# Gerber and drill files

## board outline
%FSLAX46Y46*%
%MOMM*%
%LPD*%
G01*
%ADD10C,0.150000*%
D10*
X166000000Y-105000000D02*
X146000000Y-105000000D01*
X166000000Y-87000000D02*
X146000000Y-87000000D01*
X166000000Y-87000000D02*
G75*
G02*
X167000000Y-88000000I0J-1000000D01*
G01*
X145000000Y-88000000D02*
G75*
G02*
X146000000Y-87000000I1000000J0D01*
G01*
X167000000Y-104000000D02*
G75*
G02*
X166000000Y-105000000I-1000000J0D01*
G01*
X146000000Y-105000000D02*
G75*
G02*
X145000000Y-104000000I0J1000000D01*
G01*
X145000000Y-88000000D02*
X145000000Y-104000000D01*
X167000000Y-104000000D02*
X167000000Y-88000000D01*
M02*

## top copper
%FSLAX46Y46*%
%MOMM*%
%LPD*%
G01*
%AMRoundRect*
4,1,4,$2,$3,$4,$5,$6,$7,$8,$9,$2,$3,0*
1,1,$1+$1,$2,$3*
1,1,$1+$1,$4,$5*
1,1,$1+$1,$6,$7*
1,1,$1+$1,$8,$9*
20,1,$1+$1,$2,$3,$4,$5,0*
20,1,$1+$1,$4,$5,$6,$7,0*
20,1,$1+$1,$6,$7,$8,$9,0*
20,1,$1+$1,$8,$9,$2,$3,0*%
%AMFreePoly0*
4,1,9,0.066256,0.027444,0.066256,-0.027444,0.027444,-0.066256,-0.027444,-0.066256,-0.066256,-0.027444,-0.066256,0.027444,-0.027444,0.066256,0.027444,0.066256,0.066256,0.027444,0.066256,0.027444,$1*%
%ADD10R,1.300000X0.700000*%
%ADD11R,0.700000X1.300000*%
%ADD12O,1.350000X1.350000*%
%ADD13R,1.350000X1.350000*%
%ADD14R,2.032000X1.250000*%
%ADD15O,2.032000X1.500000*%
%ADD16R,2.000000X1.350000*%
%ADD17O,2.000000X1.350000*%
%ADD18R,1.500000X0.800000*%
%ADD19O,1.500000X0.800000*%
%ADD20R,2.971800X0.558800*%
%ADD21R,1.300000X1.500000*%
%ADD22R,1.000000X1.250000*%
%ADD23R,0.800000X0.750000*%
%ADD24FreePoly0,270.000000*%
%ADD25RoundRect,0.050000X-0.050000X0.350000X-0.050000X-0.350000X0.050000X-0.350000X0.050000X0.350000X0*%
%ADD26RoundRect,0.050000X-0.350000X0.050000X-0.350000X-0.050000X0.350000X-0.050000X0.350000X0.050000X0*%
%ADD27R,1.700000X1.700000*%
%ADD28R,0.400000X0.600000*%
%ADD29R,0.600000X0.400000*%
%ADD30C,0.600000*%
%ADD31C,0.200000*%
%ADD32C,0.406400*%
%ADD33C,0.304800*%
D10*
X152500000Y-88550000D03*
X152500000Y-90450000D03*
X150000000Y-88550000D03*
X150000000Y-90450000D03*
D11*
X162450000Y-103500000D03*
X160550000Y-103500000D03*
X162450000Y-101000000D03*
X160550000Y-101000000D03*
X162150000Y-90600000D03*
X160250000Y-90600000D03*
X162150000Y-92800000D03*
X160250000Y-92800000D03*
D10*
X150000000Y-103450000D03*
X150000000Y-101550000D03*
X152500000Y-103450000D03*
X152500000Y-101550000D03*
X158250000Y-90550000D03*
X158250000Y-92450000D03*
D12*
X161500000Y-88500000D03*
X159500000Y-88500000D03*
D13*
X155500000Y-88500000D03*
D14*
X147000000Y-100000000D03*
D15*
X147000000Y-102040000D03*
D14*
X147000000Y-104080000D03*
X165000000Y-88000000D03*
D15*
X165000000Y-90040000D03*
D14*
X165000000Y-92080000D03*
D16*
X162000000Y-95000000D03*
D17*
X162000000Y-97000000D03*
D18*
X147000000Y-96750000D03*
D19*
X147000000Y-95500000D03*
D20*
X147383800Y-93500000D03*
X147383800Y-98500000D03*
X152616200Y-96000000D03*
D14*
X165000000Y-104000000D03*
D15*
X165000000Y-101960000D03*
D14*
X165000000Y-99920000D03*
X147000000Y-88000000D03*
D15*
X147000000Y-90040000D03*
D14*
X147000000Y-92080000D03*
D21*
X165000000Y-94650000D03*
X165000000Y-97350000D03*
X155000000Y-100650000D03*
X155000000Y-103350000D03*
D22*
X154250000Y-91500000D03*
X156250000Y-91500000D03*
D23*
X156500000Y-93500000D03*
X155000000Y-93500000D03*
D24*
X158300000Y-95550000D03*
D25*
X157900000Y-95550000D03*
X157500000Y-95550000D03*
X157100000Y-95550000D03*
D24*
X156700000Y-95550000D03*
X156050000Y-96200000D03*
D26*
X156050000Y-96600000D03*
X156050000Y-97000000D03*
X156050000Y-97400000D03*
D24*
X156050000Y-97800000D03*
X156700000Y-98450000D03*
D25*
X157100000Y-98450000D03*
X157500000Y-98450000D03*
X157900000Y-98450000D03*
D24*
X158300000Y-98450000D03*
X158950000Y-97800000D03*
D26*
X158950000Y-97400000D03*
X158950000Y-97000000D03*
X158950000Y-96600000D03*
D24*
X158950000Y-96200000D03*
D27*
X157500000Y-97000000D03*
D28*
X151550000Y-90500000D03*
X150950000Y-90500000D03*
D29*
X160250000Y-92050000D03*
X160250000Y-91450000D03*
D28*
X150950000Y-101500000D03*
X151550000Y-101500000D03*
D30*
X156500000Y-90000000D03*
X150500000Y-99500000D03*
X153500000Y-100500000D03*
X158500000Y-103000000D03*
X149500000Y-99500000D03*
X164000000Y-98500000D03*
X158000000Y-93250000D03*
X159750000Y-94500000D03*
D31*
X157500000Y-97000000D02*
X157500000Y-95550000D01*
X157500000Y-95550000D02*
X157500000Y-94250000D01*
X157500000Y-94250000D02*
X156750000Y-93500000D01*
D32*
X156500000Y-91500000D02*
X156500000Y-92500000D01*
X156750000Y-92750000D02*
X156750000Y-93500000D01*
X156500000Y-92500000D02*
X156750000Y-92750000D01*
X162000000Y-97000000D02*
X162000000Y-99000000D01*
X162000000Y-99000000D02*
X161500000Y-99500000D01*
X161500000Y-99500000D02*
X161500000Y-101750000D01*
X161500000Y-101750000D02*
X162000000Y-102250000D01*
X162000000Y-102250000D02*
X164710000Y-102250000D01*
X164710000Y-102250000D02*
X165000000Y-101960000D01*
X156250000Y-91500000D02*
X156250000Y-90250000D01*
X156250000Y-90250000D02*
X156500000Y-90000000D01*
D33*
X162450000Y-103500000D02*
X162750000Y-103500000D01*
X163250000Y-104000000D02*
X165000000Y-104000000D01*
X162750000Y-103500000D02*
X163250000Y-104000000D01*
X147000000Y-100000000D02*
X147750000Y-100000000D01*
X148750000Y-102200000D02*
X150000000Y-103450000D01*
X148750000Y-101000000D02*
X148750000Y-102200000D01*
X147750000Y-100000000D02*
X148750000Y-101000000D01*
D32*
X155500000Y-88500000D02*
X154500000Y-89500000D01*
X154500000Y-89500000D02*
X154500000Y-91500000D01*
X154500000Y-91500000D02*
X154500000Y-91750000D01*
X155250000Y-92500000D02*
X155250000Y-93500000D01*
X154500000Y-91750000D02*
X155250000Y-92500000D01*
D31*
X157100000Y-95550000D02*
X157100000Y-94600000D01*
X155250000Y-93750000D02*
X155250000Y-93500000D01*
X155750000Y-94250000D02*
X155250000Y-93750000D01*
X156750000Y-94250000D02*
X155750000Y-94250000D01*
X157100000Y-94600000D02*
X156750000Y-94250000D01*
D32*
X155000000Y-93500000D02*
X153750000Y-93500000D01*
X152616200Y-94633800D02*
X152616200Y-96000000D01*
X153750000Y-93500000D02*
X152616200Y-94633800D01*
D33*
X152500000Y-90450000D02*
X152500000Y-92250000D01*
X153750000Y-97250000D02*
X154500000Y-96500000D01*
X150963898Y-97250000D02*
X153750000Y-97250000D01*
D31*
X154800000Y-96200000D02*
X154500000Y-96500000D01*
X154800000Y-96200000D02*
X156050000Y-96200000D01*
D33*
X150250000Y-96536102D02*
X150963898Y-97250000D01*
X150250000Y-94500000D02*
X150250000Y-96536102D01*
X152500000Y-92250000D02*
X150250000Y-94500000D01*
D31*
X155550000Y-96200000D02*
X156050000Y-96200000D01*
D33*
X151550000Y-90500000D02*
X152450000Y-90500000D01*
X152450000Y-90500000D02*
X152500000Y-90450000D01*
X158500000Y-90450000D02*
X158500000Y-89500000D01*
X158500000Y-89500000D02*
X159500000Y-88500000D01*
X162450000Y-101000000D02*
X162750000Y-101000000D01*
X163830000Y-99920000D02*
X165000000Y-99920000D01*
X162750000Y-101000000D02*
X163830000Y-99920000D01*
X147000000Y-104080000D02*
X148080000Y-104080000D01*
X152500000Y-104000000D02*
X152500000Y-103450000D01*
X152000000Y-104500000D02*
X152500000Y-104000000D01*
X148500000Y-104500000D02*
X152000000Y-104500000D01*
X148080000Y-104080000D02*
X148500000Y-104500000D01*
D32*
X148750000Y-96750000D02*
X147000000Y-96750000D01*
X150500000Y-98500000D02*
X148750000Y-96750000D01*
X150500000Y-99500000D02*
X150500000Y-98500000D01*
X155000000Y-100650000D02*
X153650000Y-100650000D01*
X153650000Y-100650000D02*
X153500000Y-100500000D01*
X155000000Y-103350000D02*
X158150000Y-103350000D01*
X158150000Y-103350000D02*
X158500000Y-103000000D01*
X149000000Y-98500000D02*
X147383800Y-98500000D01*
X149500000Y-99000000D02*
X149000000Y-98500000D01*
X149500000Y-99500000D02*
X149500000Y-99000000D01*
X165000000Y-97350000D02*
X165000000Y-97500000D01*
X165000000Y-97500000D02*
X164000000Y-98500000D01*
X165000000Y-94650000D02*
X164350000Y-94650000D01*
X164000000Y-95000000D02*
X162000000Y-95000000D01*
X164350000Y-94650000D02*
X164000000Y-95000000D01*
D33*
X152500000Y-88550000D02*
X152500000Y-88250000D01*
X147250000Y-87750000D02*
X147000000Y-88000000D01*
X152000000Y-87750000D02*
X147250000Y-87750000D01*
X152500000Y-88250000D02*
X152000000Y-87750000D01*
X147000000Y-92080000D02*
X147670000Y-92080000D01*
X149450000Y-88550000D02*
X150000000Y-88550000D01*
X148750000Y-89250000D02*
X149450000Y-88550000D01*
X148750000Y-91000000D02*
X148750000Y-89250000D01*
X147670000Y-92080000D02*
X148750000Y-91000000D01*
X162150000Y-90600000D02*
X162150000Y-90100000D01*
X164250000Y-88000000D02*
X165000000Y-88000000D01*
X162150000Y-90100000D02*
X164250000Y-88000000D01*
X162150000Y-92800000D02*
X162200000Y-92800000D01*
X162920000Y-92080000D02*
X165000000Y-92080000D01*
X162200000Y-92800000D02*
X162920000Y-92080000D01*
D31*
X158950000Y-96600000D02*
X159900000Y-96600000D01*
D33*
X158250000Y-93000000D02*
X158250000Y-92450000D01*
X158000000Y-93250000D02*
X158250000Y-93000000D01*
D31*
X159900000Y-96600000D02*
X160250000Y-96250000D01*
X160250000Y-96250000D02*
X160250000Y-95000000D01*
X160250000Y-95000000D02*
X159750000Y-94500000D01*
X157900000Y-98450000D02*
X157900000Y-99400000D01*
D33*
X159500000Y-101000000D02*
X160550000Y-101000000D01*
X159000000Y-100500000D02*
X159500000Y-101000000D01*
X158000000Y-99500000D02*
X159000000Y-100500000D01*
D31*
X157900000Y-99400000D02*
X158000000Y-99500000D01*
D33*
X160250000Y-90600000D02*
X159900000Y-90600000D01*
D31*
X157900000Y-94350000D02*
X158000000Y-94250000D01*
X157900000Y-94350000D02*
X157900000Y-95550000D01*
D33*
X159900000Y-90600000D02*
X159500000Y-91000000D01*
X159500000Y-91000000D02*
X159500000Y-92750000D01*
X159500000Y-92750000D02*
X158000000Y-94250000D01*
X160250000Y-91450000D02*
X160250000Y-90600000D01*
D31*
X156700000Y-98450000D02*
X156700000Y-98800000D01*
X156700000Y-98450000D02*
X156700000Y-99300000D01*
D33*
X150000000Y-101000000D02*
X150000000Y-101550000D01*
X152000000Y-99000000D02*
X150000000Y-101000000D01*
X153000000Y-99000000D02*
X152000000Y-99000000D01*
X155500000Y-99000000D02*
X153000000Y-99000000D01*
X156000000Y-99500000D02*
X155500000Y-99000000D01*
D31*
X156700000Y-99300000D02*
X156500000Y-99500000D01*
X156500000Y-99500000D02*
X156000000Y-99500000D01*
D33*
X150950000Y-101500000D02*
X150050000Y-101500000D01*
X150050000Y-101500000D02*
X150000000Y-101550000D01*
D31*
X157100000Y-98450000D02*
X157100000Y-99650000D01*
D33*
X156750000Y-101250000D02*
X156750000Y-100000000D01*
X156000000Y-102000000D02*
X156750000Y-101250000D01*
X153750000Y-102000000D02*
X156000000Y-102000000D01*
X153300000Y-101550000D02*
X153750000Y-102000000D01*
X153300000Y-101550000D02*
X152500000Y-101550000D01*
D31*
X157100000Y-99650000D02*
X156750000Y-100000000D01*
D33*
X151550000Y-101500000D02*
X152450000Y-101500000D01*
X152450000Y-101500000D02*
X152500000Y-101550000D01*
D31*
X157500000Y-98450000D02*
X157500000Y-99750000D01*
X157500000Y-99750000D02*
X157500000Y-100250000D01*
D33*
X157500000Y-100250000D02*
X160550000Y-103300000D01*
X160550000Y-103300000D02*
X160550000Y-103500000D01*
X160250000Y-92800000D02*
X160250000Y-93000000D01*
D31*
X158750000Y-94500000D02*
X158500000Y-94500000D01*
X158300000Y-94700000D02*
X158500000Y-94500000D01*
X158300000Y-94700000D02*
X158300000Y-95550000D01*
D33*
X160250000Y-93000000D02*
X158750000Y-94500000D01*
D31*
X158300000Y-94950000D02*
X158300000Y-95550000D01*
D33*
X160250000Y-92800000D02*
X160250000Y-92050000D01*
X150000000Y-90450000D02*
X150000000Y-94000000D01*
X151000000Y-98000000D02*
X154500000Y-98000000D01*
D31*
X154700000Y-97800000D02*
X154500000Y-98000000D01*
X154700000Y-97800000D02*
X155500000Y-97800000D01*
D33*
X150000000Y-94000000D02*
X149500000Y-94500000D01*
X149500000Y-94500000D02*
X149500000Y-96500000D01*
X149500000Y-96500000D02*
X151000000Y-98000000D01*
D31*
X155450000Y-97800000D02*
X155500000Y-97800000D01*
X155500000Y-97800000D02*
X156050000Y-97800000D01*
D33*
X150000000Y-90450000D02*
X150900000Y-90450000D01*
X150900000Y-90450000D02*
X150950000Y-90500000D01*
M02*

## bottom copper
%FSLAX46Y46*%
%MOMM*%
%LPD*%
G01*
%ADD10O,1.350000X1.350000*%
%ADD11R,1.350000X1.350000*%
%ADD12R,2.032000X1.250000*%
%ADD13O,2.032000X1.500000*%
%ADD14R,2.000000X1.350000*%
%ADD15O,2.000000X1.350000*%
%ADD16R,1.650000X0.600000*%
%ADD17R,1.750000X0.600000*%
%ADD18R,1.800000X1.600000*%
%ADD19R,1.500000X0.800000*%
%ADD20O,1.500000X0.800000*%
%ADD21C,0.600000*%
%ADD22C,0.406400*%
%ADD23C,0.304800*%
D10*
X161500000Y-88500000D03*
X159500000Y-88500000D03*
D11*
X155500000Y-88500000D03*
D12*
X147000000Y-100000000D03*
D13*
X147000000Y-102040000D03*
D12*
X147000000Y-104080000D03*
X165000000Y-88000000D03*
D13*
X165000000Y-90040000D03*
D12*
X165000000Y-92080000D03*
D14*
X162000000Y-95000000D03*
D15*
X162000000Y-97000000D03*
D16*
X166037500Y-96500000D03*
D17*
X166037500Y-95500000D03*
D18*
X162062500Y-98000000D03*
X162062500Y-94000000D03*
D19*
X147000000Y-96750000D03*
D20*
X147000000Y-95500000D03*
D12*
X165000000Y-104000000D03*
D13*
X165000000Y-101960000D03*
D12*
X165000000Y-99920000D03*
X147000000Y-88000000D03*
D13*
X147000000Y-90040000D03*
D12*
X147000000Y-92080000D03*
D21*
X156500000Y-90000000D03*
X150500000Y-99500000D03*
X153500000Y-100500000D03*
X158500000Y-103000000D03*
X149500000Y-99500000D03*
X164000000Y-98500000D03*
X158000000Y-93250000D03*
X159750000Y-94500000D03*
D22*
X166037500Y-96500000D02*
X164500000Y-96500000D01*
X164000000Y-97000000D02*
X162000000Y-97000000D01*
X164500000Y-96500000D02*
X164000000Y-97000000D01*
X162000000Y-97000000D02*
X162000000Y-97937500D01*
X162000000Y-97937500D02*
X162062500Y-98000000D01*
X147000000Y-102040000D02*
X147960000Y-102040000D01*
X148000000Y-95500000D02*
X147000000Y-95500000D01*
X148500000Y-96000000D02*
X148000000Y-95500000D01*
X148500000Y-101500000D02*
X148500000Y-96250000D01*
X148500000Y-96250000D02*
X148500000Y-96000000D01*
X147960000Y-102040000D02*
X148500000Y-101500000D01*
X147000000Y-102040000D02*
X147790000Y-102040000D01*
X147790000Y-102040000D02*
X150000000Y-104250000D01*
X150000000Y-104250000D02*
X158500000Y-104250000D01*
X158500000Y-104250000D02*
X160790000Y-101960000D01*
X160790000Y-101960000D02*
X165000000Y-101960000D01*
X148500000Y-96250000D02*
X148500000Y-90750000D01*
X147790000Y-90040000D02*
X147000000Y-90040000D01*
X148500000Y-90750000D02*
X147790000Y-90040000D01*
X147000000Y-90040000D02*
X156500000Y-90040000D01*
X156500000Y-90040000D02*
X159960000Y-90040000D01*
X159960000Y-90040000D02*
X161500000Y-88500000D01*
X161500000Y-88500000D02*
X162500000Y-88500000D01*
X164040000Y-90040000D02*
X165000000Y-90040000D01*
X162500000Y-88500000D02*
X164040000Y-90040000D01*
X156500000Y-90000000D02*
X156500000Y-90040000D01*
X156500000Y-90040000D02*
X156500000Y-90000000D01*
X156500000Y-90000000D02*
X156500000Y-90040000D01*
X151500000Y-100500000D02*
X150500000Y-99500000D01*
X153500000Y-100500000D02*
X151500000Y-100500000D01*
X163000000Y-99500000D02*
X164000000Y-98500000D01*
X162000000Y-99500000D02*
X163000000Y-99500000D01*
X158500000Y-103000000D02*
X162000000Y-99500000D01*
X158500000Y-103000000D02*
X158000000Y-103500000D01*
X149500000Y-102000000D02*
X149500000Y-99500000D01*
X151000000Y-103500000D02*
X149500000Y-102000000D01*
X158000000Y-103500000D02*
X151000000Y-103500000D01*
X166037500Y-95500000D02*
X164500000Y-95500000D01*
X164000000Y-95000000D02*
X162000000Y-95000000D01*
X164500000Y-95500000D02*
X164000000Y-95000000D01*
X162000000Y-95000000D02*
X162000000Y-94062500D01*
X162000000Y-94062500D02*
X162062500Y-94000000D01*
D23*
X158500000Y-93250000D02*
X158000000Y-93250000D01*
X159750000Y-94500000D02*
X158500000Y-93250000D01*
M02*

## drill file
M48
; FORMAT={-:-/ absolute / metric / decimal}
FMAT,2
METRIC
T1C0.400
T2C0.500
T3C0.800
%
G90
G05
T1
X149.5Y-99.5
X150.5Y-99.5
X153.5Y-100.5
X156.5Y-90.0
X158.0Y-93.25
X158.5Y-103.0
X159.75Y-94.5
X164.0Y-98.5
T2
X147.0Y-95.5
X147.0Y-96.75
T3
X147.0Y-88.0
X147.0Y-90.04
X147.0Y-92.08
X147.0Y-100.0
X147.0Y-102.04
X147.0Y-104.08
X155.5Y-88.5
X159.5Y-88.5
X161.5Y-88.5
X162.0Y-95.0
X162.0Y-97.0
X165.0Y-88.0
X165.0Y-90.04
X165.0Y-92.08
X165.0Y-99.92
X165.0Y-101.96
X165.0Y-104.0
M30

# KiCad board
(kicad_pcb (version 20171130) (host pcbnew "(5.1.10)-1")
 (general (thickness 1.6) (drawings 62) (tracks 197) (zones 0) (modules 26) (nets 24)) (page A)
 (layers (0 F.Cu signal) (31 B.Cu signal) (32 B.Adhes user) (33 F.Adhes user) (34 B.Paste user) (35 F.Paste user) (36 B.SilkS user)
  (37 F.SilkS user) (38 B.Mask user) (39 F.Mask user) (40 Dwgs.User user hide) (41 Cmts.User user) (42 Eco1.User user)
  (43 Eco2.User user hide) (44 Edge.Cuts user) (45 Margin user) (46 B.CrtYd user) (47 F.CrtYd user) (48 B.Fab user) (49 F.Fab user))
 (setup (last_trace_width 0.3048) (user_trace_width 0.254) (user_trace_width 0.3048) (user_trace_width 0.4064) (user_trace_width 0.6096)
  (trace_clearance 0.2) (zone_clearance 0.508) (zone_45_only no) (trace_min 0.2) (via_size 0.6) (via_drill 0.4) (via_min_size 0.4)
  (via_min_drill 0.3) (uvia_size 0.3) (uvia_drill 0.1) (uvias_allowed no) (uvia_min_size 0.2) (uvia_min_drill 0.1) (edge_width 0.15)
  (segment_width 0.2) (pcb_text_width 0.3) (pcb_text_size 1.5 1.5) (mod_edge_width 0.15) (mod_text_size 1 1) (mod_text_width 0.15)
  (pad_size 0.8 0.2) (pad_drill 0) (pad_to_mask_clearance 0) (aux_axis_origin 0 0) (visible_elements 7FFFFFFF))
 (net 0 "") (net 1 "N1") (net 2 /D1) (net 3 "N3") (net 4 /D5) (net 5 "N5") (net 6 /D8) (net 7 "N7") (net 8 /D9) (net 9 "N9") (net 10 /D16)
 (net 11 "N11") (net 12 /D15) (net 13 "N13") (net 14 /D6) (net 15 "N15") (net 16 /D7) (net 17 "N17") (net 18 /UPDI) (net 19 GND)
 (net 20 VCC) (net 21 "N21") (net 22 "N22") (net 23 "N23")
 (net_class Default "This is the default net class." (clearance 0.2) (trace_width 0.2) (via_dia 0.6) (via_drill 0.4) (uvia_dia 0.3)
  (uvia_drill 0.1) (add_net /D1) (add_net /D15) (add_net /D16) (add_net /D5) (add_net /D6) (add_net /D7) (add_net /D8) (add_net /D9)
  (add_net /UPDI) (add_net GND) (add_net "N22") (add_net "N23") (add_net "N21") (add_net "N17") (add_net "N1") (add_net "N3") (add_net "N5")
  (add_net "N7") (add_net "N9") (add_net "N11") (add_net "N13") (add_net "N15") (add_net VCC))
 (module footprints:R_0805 (layer F.Cu) (at 152.5 89.5 90)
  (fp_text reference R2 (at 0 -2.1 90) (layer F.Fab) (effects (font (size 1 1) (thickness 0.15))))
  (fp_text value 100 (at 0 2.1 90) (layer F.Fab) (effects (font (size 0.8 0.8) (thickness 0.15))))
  (pad 2 smd rect (at 0.95 0 90) (size 0.7 1.3) (layers F.Cu F.Paste F.Mask) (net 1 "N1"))
  (pad 1 smd rect (at -0.95 0 90) (size 0.7 1.3) (layers F.Cu F.Paste F.Mask) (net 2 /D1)))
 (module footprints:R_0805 (layer F.Cu) (at 150 89.5 90)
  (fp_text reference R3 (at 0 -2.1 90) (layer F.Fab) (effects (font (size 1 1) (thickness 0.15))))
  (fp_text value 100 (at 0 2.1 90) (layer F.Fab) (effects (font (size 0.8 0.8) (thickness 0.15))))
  (pad 2 smd rect (at 0.95 0 90) (size 0.7 1.3) (layers F.Cu F.Paste F.Mask) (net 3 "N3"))
  (pad 1 smd rect (at -0.95 0 90) (size 0.7 1.3) (layers F.Cu F.Paste F.Mask) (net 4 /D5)))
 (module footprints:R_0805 (layer F.Cu) (at 161.5 103.5)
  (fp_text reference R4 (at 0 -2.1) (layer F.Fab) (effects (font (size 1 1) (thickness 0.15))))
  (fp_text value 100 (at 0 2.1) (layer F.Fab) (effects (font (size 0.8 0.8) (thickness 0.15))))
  (pad 2 smd rect (at 0.95 0) (size 0.7 1.3) (layers F.Cu F.Paste F.Mask) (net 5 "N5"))
  (pad 1 smd rect (at -0.95 0) (size 0.7 1.3) (layers F.Cu F.Paste F.Mask) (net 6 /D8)))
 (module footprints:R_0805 (layer F.Cu) (at 161.5 101)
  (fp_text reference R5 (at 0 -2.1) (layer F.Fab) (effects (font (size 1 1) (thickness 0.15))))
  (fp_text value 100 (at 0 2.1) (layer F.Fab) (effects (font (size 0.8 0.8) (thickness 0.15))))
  (pad 2 smd rect (at 0.95 0) (size 0.7 1.3) (layers F.Cu F.Paste F.Mask) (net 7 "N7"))
  (pad 1 smd rect (at -0.95 0) (size 0.7 1.3) (layers F.Cu F.Paste F.Mask) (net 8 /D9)))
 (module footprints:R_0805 (layer F.Cu) (at 161.2 90.6)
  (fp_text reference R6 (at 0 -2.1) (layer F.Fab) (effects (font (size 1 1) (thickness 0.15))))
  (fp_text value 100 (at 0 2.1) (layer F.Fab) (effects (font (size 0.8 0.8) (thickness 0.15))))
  (pad 2 smd rect (at 0.95 0) (size 0.7 1.3) (layers F.Cu F.Paste F.Mask) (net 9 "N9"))
  (pad 1 smd rect (at -0.95 0) (size 0.7 1.3) (layers F.Cu F.Paste F.Mask) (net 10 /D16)))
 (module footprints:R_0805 (layer F.Cu) (at 161.2 92.8)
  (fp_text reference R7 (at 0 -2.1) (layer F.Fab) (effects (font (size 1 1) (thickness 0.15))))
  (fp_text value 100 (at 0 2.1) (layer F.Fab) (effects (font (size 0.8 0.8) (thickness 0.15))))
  (pad 2 smd rect (at 0.95 0) (size 0.7 1.3) (layers F.Cu F.Paste F.Mask) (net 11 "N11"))
  (pad 1 smd rect (at -0.95 0) (size 0.7 1.3) (layers F.Cu F.Paste F.Mask) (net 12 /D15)))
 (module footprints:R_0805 (layer F.Cu) (at 150 102.5 270)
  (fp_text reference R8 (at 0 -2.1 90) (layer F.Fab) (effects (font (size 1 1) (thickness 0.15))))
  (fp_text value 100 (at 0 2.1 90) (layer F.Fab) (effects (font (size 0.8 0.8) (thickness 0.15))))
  (pad 2 smd rect (at 0.95 0 270) (size 0.7 1.3) (layers F.Cu F.Paste F.Mask) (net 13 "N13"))
  (pad 1 smd rect (at -0.95 0 270) (size 0.7 1.3) (layers F.Cu F.Paste F.Mask) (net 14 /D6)))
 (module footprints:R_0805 (layer F.Cu) (at 152.5 102.5 270)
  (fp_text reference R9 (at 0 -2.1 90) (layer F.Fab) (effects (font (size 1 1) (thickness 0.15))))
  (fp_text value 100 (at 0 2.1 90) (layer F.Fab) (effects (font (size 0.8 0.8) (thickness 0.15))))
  (pad 2 smd rect (at 0.95 0 270) (size 0.7 1.3) (layers F.Cu F.Paste F.Mask) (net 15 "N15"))
  (pad 1 smd rect (at -0.95 0 270) (size 0.7 1.3) (layers F.Cu F.Paste F.Mask) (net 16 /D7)))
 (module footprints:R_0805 (layer F.Cu) (at 158.25 91.5 90)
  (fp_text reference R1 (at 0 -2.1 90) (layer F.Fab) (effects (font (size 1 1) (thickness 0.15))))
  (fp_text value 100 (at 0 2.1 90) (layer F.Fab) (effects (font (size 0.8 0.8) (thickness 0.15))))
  (pad 2 smd rect (at 0.95 0 90) (size 0.7 1.3) (layers F.Cu F.Paste F.Mask) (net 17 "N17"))
  (pad 1 smd rect (at -0.95 0 90) (size 0.7 1.3) (layers F.Cu F.Paste F.Mask) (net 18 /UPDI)))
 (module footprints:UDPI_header (layer B.Cu) (at 155.5 88.5 270)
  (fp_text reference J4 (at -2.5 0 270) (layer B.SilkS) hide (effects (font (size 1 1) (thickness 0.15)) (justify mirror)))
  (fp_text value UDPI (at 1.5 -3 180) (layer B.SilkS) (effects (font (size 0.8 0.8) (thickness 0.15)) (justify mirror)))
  (pad 4 thru_hole oval (at 0 -6 270) (size 1.35 1.35) (drill 0.8) (layers *.Cu *.Mask) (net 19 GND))
  (pad 3 thru_hole oval (at 0 -4 270) (size 1.35 1.35) (drill 0.8) (layers *.Cu *.Mask) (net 17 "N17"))
  (pad 1 thru_hole rect (at 0 0 270) (size 1.35 1.35) (drill 0.8) (layers *.Cu *.Mask) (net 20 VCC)))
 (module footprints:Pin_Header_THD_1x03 (layer F.Cu) (at 147 100)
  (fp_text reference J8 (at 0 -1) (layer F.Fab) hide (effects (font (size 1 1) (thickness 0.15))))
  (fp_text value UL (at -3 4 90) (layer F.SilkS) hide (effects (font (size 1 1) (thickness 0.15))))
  (pad 1 thru_hole rect (at 0 0) (size 2.032 1.25) (drill 0.8) (layers *.Cu *.Mask F.SilkS) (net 13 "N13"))
  (pad 2 thru_hole oval (at 0 2.04) (size 2.032 1.5) (drill 0.8) (layers *.Cu *.Mask F.SilkS) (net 19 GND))
  (pad 3 thru_hole rect (at 0 4.08) (size 2.032 1.25) (drill 0.8) (layers *.Cu *.Mask F.SilkS) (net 15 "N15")))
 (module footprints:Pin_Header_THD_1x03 (layer F.Cu) (at 165 88)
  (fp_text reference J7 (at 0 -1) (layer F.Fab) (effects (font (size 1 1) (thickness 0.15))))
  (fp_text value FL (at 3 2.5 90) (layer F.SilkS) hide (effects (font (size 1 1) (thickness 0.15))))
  (pad 1 thru_hole rect (at 0 0) (size 2.032 1.25) (drill 0.8) (layers *.Cu *.Mask F.SilkS) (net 9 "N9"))
  (pad 2 thru_hole oval (at 0 2.04) (size 2.032 1.5) (drill 0.8) (layers *.Cu *.Mask F.SilkS) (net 19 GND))
  (pad 3 thru_hole rect (at 0 4.08) (size 2.032 1.25) (drill 0.8) (layers *.Cu *.Mask F.SilkS) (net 11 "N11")))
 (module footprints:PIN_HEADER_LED (layer B.Cu) (at 162 95 180)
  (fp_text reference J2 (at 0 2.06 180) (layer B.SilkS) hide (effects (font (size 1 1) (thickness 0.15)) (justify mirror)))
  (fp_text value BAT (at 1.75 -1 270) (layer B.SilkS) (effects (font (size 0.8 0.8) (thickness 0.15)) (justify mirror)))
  (pad 1 thru_hole rect (at 0 0 180) (size 2 1.35) (drill 0.8) (layers *.Cu *.Mask) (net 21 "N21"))
  (pad 2 thru_hole oval (at 0 -2 180) (size 2 1.35) (drill 0.8) (layers *.Cu *.Mask) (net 19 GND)))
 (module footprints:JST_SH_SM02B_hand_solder (layer B.Cu) (at 164 96 90)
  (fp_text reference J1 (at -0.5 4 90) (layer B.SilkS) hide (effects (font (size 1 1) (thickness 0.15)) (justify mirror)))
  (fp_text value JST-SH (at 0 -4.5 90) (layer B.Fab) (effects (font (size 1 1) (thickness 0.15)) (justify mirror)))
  (pad 1 smd rect (at -0.5 2.0375 90) (size 0.6 1.65) (layers B.Cu B.Paste B.Mask) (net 19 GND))
  (pad 2 smd rect (at 0.5 2.0375 90) (size 0.6 1.75) (layers B.Cu B.Paste B.Mask) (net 21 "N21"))
  (pad 1 smd rect (at -2 -1.9375 90) (size 1.6 1.8) (layers B.Cu B.Paste B.Mask) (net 19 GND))
  (pad 2 smd rect (at 2 -1.9375 90) (size 1.6 1.8) (layers B.Cu B.Paste B.Mask) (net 21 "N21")))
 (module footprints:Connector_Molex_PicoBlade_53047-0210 (layer F.Cu) (at 147 96.75 90)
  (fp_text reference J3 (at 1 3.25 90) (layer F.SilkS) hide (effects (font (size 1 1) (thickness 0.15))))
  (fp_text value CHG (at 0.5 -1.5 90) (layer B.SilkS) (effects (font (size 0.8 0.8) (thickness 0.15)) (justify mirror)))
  (pad 1 thru_hole rect (at 0 0 90) (size 0.8 1.5) (drill 0.5) (layers *.Cu *.Mask F.SilkS) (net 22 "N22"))
  (pad 2 thru_hole oval (at 1.25 0 90) (size 0.8 1.5) (drill 0.5) (layers *.Cu *.Mask F.SilkS) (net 19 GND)))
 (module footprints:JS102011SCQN (layer F.Cu) (at 150 96)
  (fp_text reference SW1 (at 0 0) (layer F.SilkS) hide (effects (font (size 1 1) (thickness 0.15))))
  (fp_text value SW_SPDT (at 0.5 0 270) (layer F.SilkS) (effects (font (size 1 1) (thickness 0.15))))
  (pad 1 smd rect (at -2.6162 -2.5) (size 2.9718 0.5588) (layers F.Cu F.Paste F.Mask))
  (pad 3 smd rect (at -2.6162 2.5) (size 2.9718 0.5588) (layers F.Cu F.Paste F.Mask) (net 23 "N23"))
  (pad 2 smd rect (at 2.6162 0) (size 2.9718 0.5588) (layers F.Cu F.Paste F.Mask) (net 20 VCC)))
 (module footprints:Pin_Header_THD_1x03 (layer F.Cu) (at 165 104 180)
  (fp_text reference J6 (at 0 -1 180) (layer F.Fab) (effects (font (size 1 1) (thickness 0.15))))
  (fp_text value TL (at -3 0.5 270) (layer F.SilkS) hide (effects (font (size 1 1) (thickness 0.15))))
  (pad 1 thru_hole rect (at 0 0 180) (size 2.032 1.25) (drill 0.8) (layers *.Cu *.Mask F.SilkS) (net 5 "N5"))
  (pad 2 thru_hole oval (at 0 2.04 180) (size 2.032 1.5) (drill 0.8) (layers *.Cu *.Mask F.SilkS) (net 19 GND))
  (pad 3 thru_hole rect (at 0 4.08 180) (size 2.032 1.25) (drill 0.8) (layers *.Cu *.Mask F.SilkS) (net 7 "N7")))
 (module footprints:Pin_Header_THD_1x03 (layer F.Cu) (at 147 88)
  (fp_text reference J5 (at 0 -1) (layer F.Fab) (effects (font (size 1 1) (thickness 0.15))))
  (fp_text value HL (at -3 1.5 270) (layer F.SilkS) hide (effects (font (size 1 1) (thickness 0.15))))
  (pad 1 thru_hole rect (at 0 0) (size 2.032 1.25) (drill 0.8) (layers *.Cu *.Mask F.SilkS) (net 1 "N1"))
  (pad 2 thru_hole oval (at 0 2.04) (size 2.032 1.5) (drill 0.8) (layers *.Cu *.Mask F.SilkS) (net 19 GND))
  (pad 3 thru_hole rect (at 0 4.08) (size 2.032 1.25) (drill 0.8) (layers *.Cu *.Mask F.SilkS) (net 3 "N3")))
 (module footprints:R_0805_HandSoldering (layer F.Cu) (at 165 96 270)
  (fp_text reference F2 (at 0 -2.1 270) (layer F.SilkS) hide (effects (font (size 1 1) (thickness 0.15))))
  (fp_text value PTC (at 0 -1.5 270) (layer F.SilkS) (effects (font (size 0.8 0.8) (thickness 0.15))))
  (pad 1 smd rect (at -1.35 0 270) (size 1.5 1.3) (layers F.Cu F.Paste F.Mask) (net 21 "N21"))
  (pad 2 smd rect (at 1.35 0 270) (size 1.5 1.3) (layers F.Cu F.Paste F.Mask) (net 23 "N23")))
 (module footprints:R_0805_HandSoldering (layer F.Cu) (at 155 102 270)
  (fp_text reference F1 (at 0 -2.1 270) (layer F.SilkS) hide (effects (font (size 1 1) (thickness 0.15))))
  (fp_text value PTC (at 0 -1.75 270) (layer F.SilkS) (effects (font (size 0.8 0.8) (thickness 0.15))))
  (pad 1 smd rect (at -1.35 0 270) (size 1.5 1.3) (layers F.Cu F.Paste F.Mask) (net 22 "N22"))
  (pad 2 smd rect (at 1.35 0 270) (size 1.5 1.3) (layers F.Cu F.Paste F.Mask) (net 23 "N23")))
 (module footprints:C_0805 (layer F.Cu) (at 155.25 91.5)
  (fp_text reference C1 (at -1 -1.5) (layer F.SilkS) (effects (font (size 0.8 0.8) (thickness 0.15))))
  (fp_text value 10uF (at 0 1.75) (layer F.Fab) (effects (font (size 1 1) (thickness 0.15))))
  (pad 1 smd rect (at -1 0) (size 1 1.25) (layers F.Cu F.Paste F.Mask) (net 20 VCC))
  (pad 2 smd rect (at 1 0) (size 1 1.25) (layers F.Cu F.Paste F.Mask) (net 19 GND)))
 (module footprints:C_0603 (layer F.Cu) (at 155.75 93.5)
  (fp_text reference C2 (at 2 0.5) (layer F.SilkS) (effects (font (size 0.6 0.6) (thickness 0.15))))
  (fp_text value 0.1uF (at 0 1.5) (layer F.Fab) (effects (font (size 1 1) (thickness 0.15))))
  (pad 2 smd rect (at 0.75 0) (size 0.8 0.75) (layers F.Cu F.Paste F.Mask) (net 19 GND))
  (pad 1 smd rect (at -0.75 0) (size 0.8 0.75) (layers F.Cu F.Paste F.Mask) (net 20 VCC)))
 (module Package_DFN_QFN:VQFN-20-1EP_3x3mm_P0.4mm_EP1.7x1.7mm (layer F.Cu) (at 157.5 97 270)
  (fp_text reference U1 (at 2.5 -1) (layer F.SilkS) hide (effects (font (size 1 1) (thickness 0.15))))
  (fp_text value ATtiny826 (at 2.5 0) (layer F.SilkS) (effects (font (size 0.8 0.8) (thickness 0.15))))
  (pad 1 smd custom (at -1.45 -0.8 270) (size 0.143431 0.143431) (layers F.Cu F.Paste F.Mask) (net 12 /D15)
   (options (clearance outline) (anchor circle)) (primitives))
  (pad 2 smd roundrect (at -1.45 -0.4 270) (size 0.8 0.2) (layers F.Cu F.Paste F.Mask) (roundrect_rratio 0.25) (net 10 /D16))
  (pad 3 smd roundrect (at -1.45 0 270) (size 0.8 0.2) (layers F.Cu F.Paste F.Mask) (roundrect_rratio 0.25) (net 19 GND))
  (pad 4 smd roundrect (at -1.45 0.4 270) (size 0.8 0.2) (layers F.Cu F.Paste F.Mask) (roundrect_rratio 0.25) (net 20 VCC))
  (pad 5 smd custom (at -1.45 0.8 270) (size 0.143431 0.143431) (layers F.Cu F.Paste F.Mask) (options (clearance outline) (anchor circle))
   (primitives))
  (pad 6 smd custom (at -0.8 1.45 270) (size 0.143431 0.143431) (layers F.Cu F.Paste F.Mask) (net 2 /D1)
   (options (clearance outline) (anchor circle)) (primitives))
  (pad 7 smd roundrect (at -0.4 1.45 270) (size 0.2 0.8) (layers F.Cu F.Paste F.Mask) (roundrect_rratio 0.25))
  (pad 8 smd roundrect (at 0 1.45 270) (size 0.2 0.8) (layers F.Cu F.Paste F.Mask) (roundrect_rratio 0.25))
  (pad 9 smd roundrect (at 0.4 1.45 270) (size 0.2 0.8) (layers F.Cu F.Paste F.Mask) (roundrect_rratio 0.25))
  (pad 10 smd custom (at 0.8 1.45 270) (size 0.143431 0.143431) (layers F.Cu F.Paste F.Mask) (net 4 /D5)
   (options (clearance outline) (anchor circle)) (primitives))
  (pad 11 smd custom (at 1.45 0.8 270) (size 0.143431 0.143431) (layers F.Cu F.Paste F.Mask) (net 14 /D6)
   (options (clearance outline) (anchor circle)) (primitives))
  (pad 12 smd roundrect (at 1.45 0.4 270) (size 0.8 0.2) (layers F.Cu F.Paste F.Mask) (roundrect_rratio 0.25) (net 16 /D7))
  (pad 13 smd roundrect (at 1.45 0 270) (size 0.8 0.2) (layers F.Cu F.Paste F.Mask) (roundrect_rratio 0.25) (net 6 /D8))
  (pad 14 smd roundrect (at 1.45 -0.4 270) (size 0.8 0.2) (layers F.Cu F.Paste F.Mask) (roundrect_rratio 0.25) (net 8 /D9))
  (pad 15 smd custom (at 1.45 -0.8 270) (size 0.143431 0.143431) (layers F.Cu F.Paste F.Mask) (options (clearance outline) (anchor circle))
   (primitives))
  (pad 16 smd custom (at 0.8 -1.45 270) (size 0.143431 0.143431) (layers F.Cu F.Paste F.Mask) (options (clearance outline) (anchor circle))
   (primitives))
  (pad 17 smd roundrect (at 0.4 -1.45 270) (size 0.2 0.8) (layers F.Cu F.Paste F.Mask) (roundrect_rratio 0.25))
  (pad 18 smd roundrect (at 0 -1.45 270) (size 0.2 0.8) (layers F.Cu F.Paste F.Mask) (roundrect_rratio 0.25))
  (pad 19 smd roundrect (at -0.4 -1.45 270) (size 0.2 0.8) (layers F.Cu F.Paste F.Mask) (roundrect_rratio 0.25) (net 18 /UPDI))
  (pad 20 smd custom (at -0.8 -1.45 270) (size 0.143431 0.143431) (layers F.Cu F.Paste F.Mask) (options (clearance outline) (anchor circle))
   (primitives))
  (pad 21 smd rect (at 0 0 270) (size 1.7 1.7) (layers F.Cu F.Mask) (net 19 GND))
  (pad "" smd roundrect (at -0.425 -0.425 270) (size 0.69 0.69) (layers F.Paste) (roundrect_rratio 0.25))
  (pad "" smd roundrect (at -0.425 0.425 270) (size 0.69 0.69) (layers F.Paste) (roundrect_rratio 0.25))
  (pad "" smd roundrect (at 0.425 -0.425 270) (size 0.69 0.69) (layers F.Paste) (roundrect_rratio 0.25))
  (pad "" smd roundrect (at 0.425 0.425 270) (size 0.69 0.69) (layers F.Paste) (roundrect_rratio 0.25)))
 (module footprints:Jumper (layer F.Cu) (at 151.25 90.5 180)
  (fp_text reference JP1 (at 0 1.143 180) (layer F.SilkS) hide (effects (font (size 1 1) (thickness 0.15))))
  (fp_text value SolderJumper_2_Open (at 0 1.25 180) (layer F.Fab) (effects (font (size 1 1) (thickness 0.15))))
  (pad 1 smd rect (at -0.3 0 180) (size 0.4 0.6) (layers F.Cu F.Paste F.Mask) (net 2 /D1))
  (pad 2 smd rect (at 0.3 0 180) (size 0.4 0.6) (layers F.Cu F.Paste F.Mask) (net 4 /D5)))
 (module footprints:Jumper (layer F.Cu) (at 160.25 91.75 270)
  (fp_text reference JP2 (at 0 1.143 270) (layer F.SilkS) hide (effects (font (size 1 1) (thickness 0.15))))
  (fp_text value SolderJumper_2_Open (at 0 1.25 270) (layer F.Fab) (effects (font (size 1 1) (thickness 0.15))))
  (pad 2 smd rect (at 0.3 0 270) (size 0.4 0.6) (layers F.Cu F.Paste F.Mask) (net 12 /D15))
  (pad 1 smd rect (at -0.3 0 270) (size 0.4 0.6) (layers F.Cu F.Paste F.Mask) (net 10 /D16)))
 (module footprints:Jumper (layer F.Cu) (at 151.25 101.5)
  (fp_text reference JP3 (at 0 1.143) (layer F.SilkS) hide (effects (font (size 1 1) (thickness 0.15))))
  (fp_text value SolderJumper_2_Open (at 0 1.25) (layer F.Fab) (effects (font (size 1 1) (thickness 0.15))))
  (pad 1 smd rect (at -0.3 0) (size 0.4 0.6) (layers F.Cu F.Paste F.Mask) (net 14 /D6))
  (pad 2 smd rect (at 0.3 0) (size 0.4 0.6) (layers F.Cu F.Paste F.Mask) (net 16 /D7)))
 (gr_line (start 166 105) (end 146 105) (angle 90) (layer Edge.Cuts) (width 0.15))
 (gr_line (start 166 87) (end 146 87) (angle 90) (layer Edge.Cuts) (width 0.15))
 (gr_arc (start 166 88) (end 166 87) (angle 90) (layer Edge.Cuts) (width 0.15))
 (gr_arc (start 146 88) (end 145 88) (angle 90) (layer Edge.Cuts) (width 0.15))
 (gr_arc (start 166 104) (end 167 104) (angle 90) (layer Edge.Cuts) (width 0.15))
 (gr_arc (start 146 104) (end 146 105) (angle 90) (layer Edge.Cuts) (width 0.15))
 (gr_line (start 145 88) (end 145 104) (angle 90) (layer Edge.Cuts) (width 0.15))
 (gr_line (start 167 104) (end 167 88) (angle 90) (layer Edge.Cuts) (width 0.15))
 (segment (start 166.0375 96.5) (end 164.5 96.5) (width 0.4064) (layer B.Cu) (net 19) (status 400010))
 (segment (start 164 97) (end 162 97) (width 0.4064) (layer B.Cu) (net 19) (status 800020))
 (segment (start 164.5 96.5) (end 164 97) (width 0.4064) (layer B.Cu) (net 19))
 (segment (start 162 97) (end 162 97.9375) (width 0.4064) (layer B.Cu) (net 19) (status C00030))
 (segment (start 162 97.9375) (end 162.0625 98) (width 0.4064) (layer B.Cu) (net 19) (status C00030))
 (segment (start 147 102.04) (end 147.96 102.04) (width 0.4064) (layer B.Cu) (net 19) (status C00030))
 (segment (start 148 95.5) (end 147 95.5) (width 0.4064) (layer B.Cu) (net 19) (status 800020))
 (segment (start 148.5 96) (end 148 95.5) (width 0.4064) (layer B.Cu) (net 19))
 (segment (start 148.5 101.5) (end 148.5 96.25) (width 0.4064) (layer B.Cu) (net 19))
 (segment (start 148.5 96.25) (end 148.5 96) (width 0.4064) (layer B.Cu) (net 19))
 (segment (start 147.96 102.04) (end 148.5 101.5) (width 0.4064) (layer B.Cu) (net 19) (status 400010))
 (segment (start 147 102.04) (end 147.79 102.04) (width 0.4064) (layer B.Cu) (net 19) (status C00030))
 (segment (start 147.79 102.04) (end 150 104.25) (width 0.4064) (layer B.Cu) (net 19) (status 400010))
 (segment (start 150 104.25) (end 158.5 104.25) (width 0.4064) (layer B.Cu) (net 19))
 (segment (start 158.5 104.25) (end 160.79 101.96) (width 0.4064) (layer B.Cu) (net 19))
 (segment (start 160.79 101.96) (end 165 101.96) (width 0.4064) (layer B.Cu) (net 19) (status 800020))
 (segment (start 148.5 96.25) (end 148.5 90.75) (width 0.4064) (layer B.Cu) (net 19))
 (segment (start 147.79 90.04) (end 147 90.04) (width 0.4064) (layer B.Cu) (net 19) (status C00030))
 (segment (start 148.5 90.75) (end 147.79 90.04) (width 0.4064) (layer B.Cu) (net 19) (status 800020))
 (segment (start 147 90.04) (end 156.5 90.04) (width 0.4064) (layer B.Cu) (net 19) (status 400010))
 (segment (start 156.5 90.04) (end 159.96 90.04) (width 0.4064) (layer B.Cu) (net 19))
 (segment (start 159.96 90.04) (end 161.5 88.5) (width 0.4064) (layer B.Cu) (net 19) (status 800020))
 (segment (start 161.5 88.5) (end 162.5 88.5) (width 0.4064) (layer B.Cu) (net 19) (status 400010))
 (segment (start 164.04 90.04) (end 165 90.04) (width 0.4064) (layer B.Cu) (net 19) (status C00030))
 (segment (start 162.5 88.5) (end 164.04 90.04) (width 0.4064) (layer B.Cu) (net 19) (status 800020))
 (segment (start 157.5 97) (end 157.5 95.55) (width 0.2) (layer F.Cu) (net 19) (status C00030))
 (segment (start 157.5 95.55) (end 157.5 94.25) (width 0.2) (layer F.Cu) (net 19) (status 400010))
 (segment (start 157.5 94.25) (end 156.75 93.5) (width 0.2) (layer F.Cu) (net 19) (status 800020))
 (segment (start 156.5 91.5) (end 156.5 92.5) (width 0.4064) (layer F.Cu) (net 19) (status 400010))
 (segment (start 156.75 92.75) (end 156.75 93.5) (width 0.4064) (layer F.Cu) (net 19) (status 800020))
 (segment (start 156.5 92.5) (end 156.75 92.75) (width 0.4064) (layer F.Cu) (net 19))
 (segment (start 162 97) (end 162 99) (width 0.4064) (layer F.Cu) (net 19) (status 400010))
 (segment (start 162 99) (end 161.5 99.5) (width 0.4064) (layer F.Cu) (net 19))
 (segment (start 161.5 99.5) (end 161.5 101.75) (width 0.4064) (layer F.Cu) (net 19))
 (segment (start 161.5 101.75) (end 162 102.25) (width 0.4064) (layer F.Cu) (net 19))
 (segment (start 162 102.25) (end 164.71 102.25) (width 0.4064) (layer F.Cu) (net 19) (status 800020))
 (segment (start 164.71 102.25) (end 165 101.96) (width 0.4064) (layer F.Cu) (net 19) (status C00030))
 (segment (start 156.25 91.5) (end 156.25 90.25) (width 0.4064) (layer F.Cu) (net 19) (status 400010))
 (via (at 156.5 90) (size 0.6) (drill 0.4) (layers F.Cu B.Cu) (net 19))
 (segment (start 156.25 90.25) (end 156.5 90) (width 0.4064) (layer F.Cu) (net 19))
 (segment (start 156.5 90) (end 156.5 90.04) (width 0.4064) (layer B.Cu) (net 19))
 (segment (start 156.5 90.04) (end 156.5 90) (width 0.4064) (layer B.Cu) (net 19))
 (segment (start 156.5 90) (end 156.5 90.04) (width 0.4064) (layer B.Cu) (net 19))
 (segment (start 162.45 103.5) (end 162.75 103.5) (width 0.3048) (layer F.Cu) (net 5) (status C00030))
 (segment (start 163.25 104) (end 165 104) (width 0.3048) (layer F.Cu) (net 5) (status 800020))
 (segment (start 162.75 103.5) (end 163.25 104) (width 0.3048) (layer F.Cu) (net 5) (status 400010))
 (segment (start 147 100) (end 147.75 100) (width 0.3048) (layer F.Cu) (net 13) (status C00030))
 (segment (start 148.75 102.2) (end 150 103.45) (width 0.3048) (layer F.Cu) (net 13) (status 800020))
 (segment (start 148.75 101) (end 148.75 102.2) (width 0.3048) (layer F.Cu) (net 13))
 (segment (start 147.75 100) (end 148.75 101) (width 0.3048) (layer F.Cu) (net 13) (status 400010))
 (segment (start 155.5 88.5) (end 154.5 89.5) (width 0.4064) (layer F.Cu) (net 20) (status 400010))
 (segment (start 154.5 89.5) (end 154.5 91.5) (width 0.4064) (layer F.Cu) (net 20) (status 800020))
 (segment (start 154.5 91.5) (end 154.5 91.75) (width 0.4064) (layer F.Cu) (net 20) (status C00030))
 (segment (start 155.25 92.5) (end 155.25 93.5) (width 0.4064) (layer F.Cu) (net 20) (status 800020))
 (segment (start 154.5 91.75) (end 155.25 92.5) (width 0.4064) (layer F.Cu) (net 20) (status 400010))
 (segment (start 157.1 95.55) (end 157.1 94.6) (width 0.2) (layer F.Cu) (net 20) (status 400010))
 (segment (start 155.25 93.75) (end 155.25 93.5) (width 0.2) (layer F.Cu) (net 20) (status C00030))
 (segment (start 155.75 94.25) (end 155.25 93.75) (width 0.2) (layer F.Cu) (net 20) (status 800020))
 (segment (start 156.75 94.25) (end 155.75 94.25) (width 0.2) (layer F.Cu) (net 20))
 (segment (start 157.1 94.6) (end 156.75 94.25) (width 0.2) (layer F.Cu) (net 20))
 (segment (start 155 93.5) (end 153.75 93.5) (width 0.4064) (layer F.Cu) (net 20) (status 400010))
 (segment (start 152.6162 94.6338) (end 152.6162 96) (width 0.4064) (layer F.Cu) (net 20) (status 800020))
 (segment (start 153.75 93.5) (end 152.6162 94.6338) (width 0.4064) (layer F.Cu) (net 20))
 (segment (start 152.5 90.45) (end 152.5 92.25) (width 0.3048) (layer F.Cu) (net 2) (status 400010))
 (segment (start 153.75 97.25) (end 154.5 96.5) (width 0.3048) (layer F.Cu) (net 2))
 (segment (start 150.963898 97.25) (end 153.75 97.25) (width 0.3048) (layer F.Cu) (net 2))
 (segment (start 154.8 96.2) (end 154.5 96.5) (width 0.2) (layer F.Cu) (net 2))
 (segment (start 154.8 96.2) (end 156.05 96.2) (width 0.2) (layer F.Cu) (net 2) (status 800020))
 (segment (start 150.25 96.536102) (end 150.963898 97.25) (width 0.3048) (layer F.Cu) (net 2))
 (segment (start 150.25 94.5) (end 150.25 96.536102) (width 0.3048) (layer F.Cu) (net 2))
 (segment (start 152.5 92.25) (end 150.25 94.5) (width 0.3048) (layer F.Cu) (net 2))
 (segment (start 155.55 96.2) (end 156.05 96.2) (width 0.2) (layer F.Cu) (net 2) (status 800020))
 (segment (start 151.55 90.5) (end 152.45 90.5) (width 0.3048) (layer F.Cu) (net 2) (status C00000))
 (segment (start 152.45 90.5) (end 152.5 90.45) (width 0.3048) (layer F.Cu) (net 2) (status C00000))
 (segment (start 158.5 90.45) (end 158.5 89.5) (width 0.3048) (layer F.Cu) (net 17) (status 400010))
 (segment (start 158.5 89.5) (end 159.5 88.5) (width 0.3048) (layer F.Cu) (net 17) (status 800020))
 (segment (start 162.45 101) (end 162.75 101) (width 0.3048) (layer F.Cu) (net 7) (status C00030))
 (segment (start 163.83 99.92) (end 165 99.92) (width 0.3048) (layer F.Cu) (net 7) (status 800020))
 (segment (start 162.75 101) (end 163.83 99.92) (width 0.3048) (layer F.Cu) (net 7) (status 400010))
 (segment (start 147 104.08) (end 148.08 104.08) (width 0.3048) (layer F.Cu) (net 15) (status 400010))
 (segment (start 152.5 104) (end 152.5 103.45) (width 0.3048) (layer F.Cu) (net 15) (status 800020))
 (segment (start 152 104.5) (end 152.5 104) (width 0.3048) (layer F.Cu) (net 15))
 (segment (start 148.5 104.5) (end 152 104.5) (width 0.3048) (layer F.Cu) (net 15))
 (segment (start 148.08 104.08) (end 148.5 104.5) (width 0.3048) (layer F.Cu) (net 15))
 (segment (start 148.75 96.75) (end 147 96.75) (width 0.4064) (layer F.Cu) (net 22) (status 800020))
 (segment (start 150.5 98.5) (end 148.75 96.75) (width 0.4064) (layer F.Cu) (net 22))
 (segment (start 150.5 99.5) (end 150.5 98.5) (width 0.4064) (layer F.Cu) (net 22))
 (via (at 150.5 99.5) (size 0.6) (drill 0.4) (layers F.Cu B.Cu) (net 22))
 (segment (start 155 100.65) (end 153.65 100.65) (width 0.4064) (layer F.Cu) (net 22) (status 400010))
 (segment (start 151.5 100.5) (end 150.5 99.5) (width 0.4064) (layer B.Cu) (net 22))
 (segment (start 153.5 100.5) (end 151.5 100.5) (width 0.4064) (layer B.Cu) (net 22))
 (via (at 153.5 100.5) (size 0.6) (drill 0.4) (layers F.Cu B.Cu) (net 22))
 (segment (start 153.65 100.65) (end 153.5 100.5) (width 0.4064) (layer F.Cu) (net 22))
 (segment (start 155 103.35) (end 158.15 103.35) (width 0.4064) (layer F.Cu) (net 23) (status 400010))
 (segment (start 163 99.5) (end 164 98.5) (width 0.4064) (layer B.Cu) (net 23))
 (segment (start 162 99.5) (end 163 99.5) (width 0.4064) (layer B.Cu) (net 23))
 (segment (start 158.5 103) (end 162 99.5) (width 0.4064) (layer B.Cu) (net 23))
 (via (at 158.5 103) (size 0.6) (drill 0.4) (layers F.Cu B.Cu) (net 23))
 (segment (start 158.15 103.35) (end 158.5 103) (width 0.4064) (layer F.Cu) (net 23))
 (segment (start 158.5 103) (end 158 103.5) (width 0.4064) (layer B.Cu) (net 23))
 (segment (start 149 98.5) (end 147.3838 98.5) (width 0.4064) (layer F.Cu) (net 23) (status 800020))
 (segment (start 149.5 99) (end 149 98.5) (width 0.4064) (layer F.Cu) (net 23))
 (segment (start 149.5 99.5) (end 149.5 99) (width 0.4064) (layer F.Cu) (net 23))
 (via (at 149.5 99.5) (size 0.6) (drill 0.4) (layers F.Cu B.Cu) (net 23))
 (segment (start 149.5 102) (end 149.5 99.5) (width 0.4064) (layer B.Cu) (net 23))
 (segment (start 151 103.5) (end 149.5 102) (width 0.4064) (layer B.Cu) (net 23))
 (segment (start 158 103.5) (end 151 103.5) (width 0.4064) (layer B.Cu) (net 23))
 (segment (start 165 97.35) (end 165 97.5) (width 0.4064) (layer F.Cu) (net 23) (status C00030))
 (via (at 164 98.5) (size 0.6) (drill 0.4) (layers F.Cu B.Cu) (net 23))
 (segment (start 165 97.5) (end 164 98.5) (width 0.4064) (layer F.Cu) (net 23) (status 400010))
 (segment (start 165 94.65) (end 164.35 94.65) (width 0.4064) (layer F.Cu) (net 21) (status C00030))
 (segment (start 164 95) (end 162 95) (width 0.4064) (layer F.Cu) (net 21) (status 800020))
 (segment (start 164.35 94.65) (end 164 95) (width 0.4064) (layer F.Cu) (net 21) (status 400010))
 (segment (start 166.0375 95.5) (end 164.5 95.5) (width 0.4064) (layer B.Cu) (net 21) (status 400010))
 (segment (start 164 95) (end 162 95) (width 0.4064) (layer B.Cu) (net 21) (status 800020))
 (segment (start 164.5 95.5) (end 164 95) (width 0.4064) (layer B.Cu) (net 21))
 (segment (start 162 95) (end 162 94.0625) (width 0.4064) (layer B.Cu) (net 21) (status C00030))
 (segment (start 162 94.0625) (end 162.0625 94) (width 0.4064) (layer B.Cu) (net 21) (status C00030))
 (segment (start 152.5 88.55) (end 152.5 88.25) (width 0.3048) (layer F.Cu) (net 1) (status C00030))
 (segment (start 147.25 87.75) (end 147 88) (width 0.3048) (layer F.Cu) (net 1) (status C00030))
 (segment (start 152 87.75) (end 147.25 87.75) (width 0.3048) (layer F.Cu) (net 1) (status 800020))
 (segment (start 152.5 88.25) (end 152 87.75) (width 0.3048) (layer F.Cu) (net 1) (status 400010))
 (segment (start 147 92.08) (end 147.67 92.08) (width 0.3048) (layer F.Cu) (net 3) (status C00030))
 (segment (start 149.45 88.55) (end 150 88.55) (width 0.3048) (layer F.Cu) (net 3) (status C00030))
 (segment (start 148.75 89.25) (end 149.45 88.55) (width 0.3048) (layer F.Cu) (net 3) (status 800020))
 (segment (start 148.75 91) (end 148.75 89.25) (width 0.3048) (layer F.Cu) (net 3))
 (segment (start 147.67 92.08) (end 148.75 91) (width 0.3048) (layer F.Cu) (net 3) (status 400010))
 (segment (start 162.15 90.6) (end 162.15 90.1) (width 0.3048) (layer F.Cu) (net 9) (status C00030))
 (segment (start 164.25 88) (end 165 88) (width 0.3048) (layer F.Cu) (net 9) (status C00030))
 (segment (start 162.15 90.1) (end 164.25 88) (width 0.3048) (layer F.Cu) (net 9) (status C00030))
 (segment (start 162.15 92.8) (end 162.2 92.8) (width 0.3048) (layer F.Cu) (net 11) (status C00030))
 (segment (start 162.92 92.08) (end 165 92.08) (width 0.3048) (layer F.Cu) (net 11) (status 800020))
 (segment (start 162.2 92.8) (end 162.92 92.08) (width 0.3048) (layer F.Cu) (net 11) (status 400010))
 (segment (start 158.95 96.6) (end 159.9 96.6) (width 0.2) (layer F.Cu) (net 18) (status 400010))
 (segment (start 158.25 93) (end 158.25 92.45) (width 0.3048) (layer F.Cu) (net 18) (status 800020))
 (segment (start 158 93.25) (end 158.25 93) (width 0.3048) (layer F.Cu) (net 18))
 (via (at 158 93.25) (size 0.6) (drill 0.4) (layers F.Cu B.Cu) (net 18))
 (segment (start 158.5 93.25) (end 158 93.25) (width 0.3048) (layer B.Cu) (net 18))
 (segment (start 159.75 94.5) (end 158.5 93.25) (width 0.3048) (layer B.Cu) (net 18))
 (via (at 159.75 94.5) (size 0.6) (drill 0.4) (layers F.Cu B.Cu) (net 18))
 (segment (start 159.9 96.6) (end 160.25 96.25) (width 0.2) (layer F.Cu) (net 18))
 (segment (start 160.25 96.25) (end 160.25 95) (width 0.2) (layer F.Cu) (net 18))
 (segment (start 160.25 95) (end 159.75 94.5) (width 0.2) (layer F.Cu) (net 18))
 (segment (start 157.9 98.45) (end 157.9 99.4) (width 0.2) (layer F.Cu) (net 8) (status 400010))
 (segment (start 159.5 101) (end 160.55 101) (width 0.3048) (layer F.Cu) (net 8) (status 800020))
 (segment (start 159 100.5) (end 159.5 101) (width 0.3048) (layer F.Cu) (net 8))
 (segment (start 158 99.5) (end 159 100.5) (width 0.3048) (layer F.Cu) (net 8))
 (segment (start 157.9 99.4) (end 158 99.5) (width 0.2) (layer F.Cu) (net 8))
 (segment (start 160.25 90.6) (end 159.9 90.6) (width 0.3048) (layer F.Cu) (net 10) (status C00030))
 (segment (start 157.9 94.35) (end 158 94.25) (width 0.2) (layer F.Cu) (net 10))
 (segment (start 157.9 94.35) (end 157.9 95.55) (width 0.2) (layer F.Cu) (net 10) (status 800020))
 (segment (start 159.9 90.6) (end 159.5 91) (width 0.3048) (layer F.Cu) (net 10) (status 400010))
 (segment (start 159.5 91) (end 159.5 92.75) (width 0.3048) (layer F.Cu) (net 10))
 (segment (start 159.5 92.75) (end 158 94.25) (width 0.3048) (layer F.Cu) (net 10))
 (segment (start 160.25 91.45) (end 160.25 90.6) (width 0.3048) (layer F.Cu) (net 10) (status C00000))
 (segment (start 156.7 98.45) (end 156.7 98.8) (width 0.2) (layer F.Cu) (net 14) (status C00030))
 (segment (start 156.7 98.45) (end 156.7 99.3) (width 0.2) (layer F.Cu) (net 14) (status 400010))
 (segment (start 150 101) (end 150 101.55) (width 0.3048) (layer F.Cu) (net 14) (status 800020))
 (segment (start 152 99) (end 150 101) (width 0.3048) (layer F.Cu) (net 14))
 (segment (start 153 99) (end 152 99) (width 0.3048) (layer F.Cu) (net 14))
 (segment (start 155.5 99) (end 153 99) (width 0.3048) (layer F.Cu) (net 14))
 (segment (start 156 99.5) (end 155.5 99) (width 0.3048) (layer F.Cu) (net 14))
 (segment (start 156.7 99.3) (end 156.5 99.5) (width 0.2) (layer F.Cu) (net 14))
 (segment (start 156.5 99.5) (end 156 99.5) (width 0.2) (layer F.Cu) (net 14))
 (segment (start 150.95 101.5) (end 150.05 101.5) (width 0.3048) (layer F.Cu) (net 14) (status C00000))
 (segment (start 150.05 101.5) (end 150 101.55) (width 0.3048) (layer F.Cu) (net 14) (status C00000))
 (segment (start 157.1 98.45) (end 157.1 99.65) (width 0.2) (layer F.Cu) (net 16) (status 400010))
 (segment (start 156.75 101.25) (end 156.75 100) (width 0.3048) (layer F.Cu) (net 16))
 (segment (start 156 102) (end 156.75 101.25) (width 0.3048) (layer F.Cu) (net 16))
 (segment (start 153.75 102) (end 156 102) (width 0.3048) (layer F.Cu) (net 16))
 (segment (start 153.3 101.55) (end 153.75 102) (width 0.3048) (layer F.Cu) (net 16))
 (segment (start 153.3 101.55) (end 152.5 101.55) (width 0.3048) (layer F.Cu) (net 16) (status 800020))
 (segment (start 157.1 99.65) (end 156.75 100) (width 0.2) (layer F.Cu) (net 16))
 (segment (start 151.55 101.5) (end 152.45 101.5) (width 0.3048) (layer F.Cu) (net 16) (status C00000))
 (segment (start 152.45 101.5) (end 152.5 101.55) (width 0.3048) (layer F.Cu) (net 16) (status C00000))
 (segment (start 157.5 98.45) (end 157.5 99.75) (width 0.2) (layer F.Cu) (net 6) (status 400010))
 (segment (start 157.5 99.75) (end 157.5 100.25) (width 0.2) (layer F.Cu) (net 6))
 (segment (start 157.5 100.25) (end 160.55 103.3) (width 0.3048) (layer F.Cu) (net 6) (status 800020))
 (segment (start 160.55 103.3) (end 160.55 103.5) (width 0.3048) (layer F.Cu) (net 6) (status C00030))
 (segment (start 160.25 92.8) (end 160.25 93) (width 0.3048) (layer F.Cu) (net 12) (status C00030))
 (segment (start 158.75 94.5) (end 158.5 94.5) (width 0.2) (layer F.Cu) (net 12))
 (segment (start 158.3 94.7) (end 158.5 94.5) (width 0.2) (layer F.Cu) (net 12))
 (segment (start 158.3 94.7) (end 158.3 95.55) (width 0.2) (layer F.Cu) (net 12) (status 800020))
 (segment (start 160.25 93) (end 158.75 94.5) (width 0.3048) (layer F.Cu) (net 12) (status 400010))
 (segment (start 158.3 94.95) (end 158.3 95.55) (width 0.2) (layer F.Cu) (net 12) (status 800020))
 (segment (start 160.25 92.8) (end 160.25 92.05) (width 0.3048) (layer F.Cu) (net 12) (status C00000))
 (segment (start 150 90.45) (end 150 94) (width 0.3048) (layer F.Cu) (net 4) (status 400010))
 (segment (start 151 98) (end 154.5 98) (width 0.3048) (layer F.Cu) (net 4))
 (segment (start 154.7 97.8) (end 154.5 98) (width 0.2) (layer F.Cu) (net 4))
 (segment (start 154.7 97.8) (end 155.5 97.8) (width 0.2) (layer F.Cu) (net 4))
 (segment (start 150 94) (end 149.5 94.5) (width 0.3048) (layer F.Cu) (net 4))
 (segment (start 149.5 94.5) (end 149.5 96.5) (width 0.3048) (layer F.Cu) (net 4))
 (segment (start 149.5 96.5) (end 151 98) (width 0.3048) (layer F.Cu) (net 4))
 (segment (start 155.45 97.8) (end 155.5 97.8) (width 0.2) (layer F.Cu) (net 4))
 (segment (start 155.5 97.8) (end 156.05 97.8) (width 0.2) (layer F.Cu) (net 4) (status 800020))
 (segment (start 150 90.45) (end 150.9 90.45) (width 0.3048) (layer F.Cu) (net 4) (status C00000))
 (segment (start 150.9 90.45) (end 150.95 90.5) (width 0.3048) (layer F.Cu) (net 4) (status C00000)))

